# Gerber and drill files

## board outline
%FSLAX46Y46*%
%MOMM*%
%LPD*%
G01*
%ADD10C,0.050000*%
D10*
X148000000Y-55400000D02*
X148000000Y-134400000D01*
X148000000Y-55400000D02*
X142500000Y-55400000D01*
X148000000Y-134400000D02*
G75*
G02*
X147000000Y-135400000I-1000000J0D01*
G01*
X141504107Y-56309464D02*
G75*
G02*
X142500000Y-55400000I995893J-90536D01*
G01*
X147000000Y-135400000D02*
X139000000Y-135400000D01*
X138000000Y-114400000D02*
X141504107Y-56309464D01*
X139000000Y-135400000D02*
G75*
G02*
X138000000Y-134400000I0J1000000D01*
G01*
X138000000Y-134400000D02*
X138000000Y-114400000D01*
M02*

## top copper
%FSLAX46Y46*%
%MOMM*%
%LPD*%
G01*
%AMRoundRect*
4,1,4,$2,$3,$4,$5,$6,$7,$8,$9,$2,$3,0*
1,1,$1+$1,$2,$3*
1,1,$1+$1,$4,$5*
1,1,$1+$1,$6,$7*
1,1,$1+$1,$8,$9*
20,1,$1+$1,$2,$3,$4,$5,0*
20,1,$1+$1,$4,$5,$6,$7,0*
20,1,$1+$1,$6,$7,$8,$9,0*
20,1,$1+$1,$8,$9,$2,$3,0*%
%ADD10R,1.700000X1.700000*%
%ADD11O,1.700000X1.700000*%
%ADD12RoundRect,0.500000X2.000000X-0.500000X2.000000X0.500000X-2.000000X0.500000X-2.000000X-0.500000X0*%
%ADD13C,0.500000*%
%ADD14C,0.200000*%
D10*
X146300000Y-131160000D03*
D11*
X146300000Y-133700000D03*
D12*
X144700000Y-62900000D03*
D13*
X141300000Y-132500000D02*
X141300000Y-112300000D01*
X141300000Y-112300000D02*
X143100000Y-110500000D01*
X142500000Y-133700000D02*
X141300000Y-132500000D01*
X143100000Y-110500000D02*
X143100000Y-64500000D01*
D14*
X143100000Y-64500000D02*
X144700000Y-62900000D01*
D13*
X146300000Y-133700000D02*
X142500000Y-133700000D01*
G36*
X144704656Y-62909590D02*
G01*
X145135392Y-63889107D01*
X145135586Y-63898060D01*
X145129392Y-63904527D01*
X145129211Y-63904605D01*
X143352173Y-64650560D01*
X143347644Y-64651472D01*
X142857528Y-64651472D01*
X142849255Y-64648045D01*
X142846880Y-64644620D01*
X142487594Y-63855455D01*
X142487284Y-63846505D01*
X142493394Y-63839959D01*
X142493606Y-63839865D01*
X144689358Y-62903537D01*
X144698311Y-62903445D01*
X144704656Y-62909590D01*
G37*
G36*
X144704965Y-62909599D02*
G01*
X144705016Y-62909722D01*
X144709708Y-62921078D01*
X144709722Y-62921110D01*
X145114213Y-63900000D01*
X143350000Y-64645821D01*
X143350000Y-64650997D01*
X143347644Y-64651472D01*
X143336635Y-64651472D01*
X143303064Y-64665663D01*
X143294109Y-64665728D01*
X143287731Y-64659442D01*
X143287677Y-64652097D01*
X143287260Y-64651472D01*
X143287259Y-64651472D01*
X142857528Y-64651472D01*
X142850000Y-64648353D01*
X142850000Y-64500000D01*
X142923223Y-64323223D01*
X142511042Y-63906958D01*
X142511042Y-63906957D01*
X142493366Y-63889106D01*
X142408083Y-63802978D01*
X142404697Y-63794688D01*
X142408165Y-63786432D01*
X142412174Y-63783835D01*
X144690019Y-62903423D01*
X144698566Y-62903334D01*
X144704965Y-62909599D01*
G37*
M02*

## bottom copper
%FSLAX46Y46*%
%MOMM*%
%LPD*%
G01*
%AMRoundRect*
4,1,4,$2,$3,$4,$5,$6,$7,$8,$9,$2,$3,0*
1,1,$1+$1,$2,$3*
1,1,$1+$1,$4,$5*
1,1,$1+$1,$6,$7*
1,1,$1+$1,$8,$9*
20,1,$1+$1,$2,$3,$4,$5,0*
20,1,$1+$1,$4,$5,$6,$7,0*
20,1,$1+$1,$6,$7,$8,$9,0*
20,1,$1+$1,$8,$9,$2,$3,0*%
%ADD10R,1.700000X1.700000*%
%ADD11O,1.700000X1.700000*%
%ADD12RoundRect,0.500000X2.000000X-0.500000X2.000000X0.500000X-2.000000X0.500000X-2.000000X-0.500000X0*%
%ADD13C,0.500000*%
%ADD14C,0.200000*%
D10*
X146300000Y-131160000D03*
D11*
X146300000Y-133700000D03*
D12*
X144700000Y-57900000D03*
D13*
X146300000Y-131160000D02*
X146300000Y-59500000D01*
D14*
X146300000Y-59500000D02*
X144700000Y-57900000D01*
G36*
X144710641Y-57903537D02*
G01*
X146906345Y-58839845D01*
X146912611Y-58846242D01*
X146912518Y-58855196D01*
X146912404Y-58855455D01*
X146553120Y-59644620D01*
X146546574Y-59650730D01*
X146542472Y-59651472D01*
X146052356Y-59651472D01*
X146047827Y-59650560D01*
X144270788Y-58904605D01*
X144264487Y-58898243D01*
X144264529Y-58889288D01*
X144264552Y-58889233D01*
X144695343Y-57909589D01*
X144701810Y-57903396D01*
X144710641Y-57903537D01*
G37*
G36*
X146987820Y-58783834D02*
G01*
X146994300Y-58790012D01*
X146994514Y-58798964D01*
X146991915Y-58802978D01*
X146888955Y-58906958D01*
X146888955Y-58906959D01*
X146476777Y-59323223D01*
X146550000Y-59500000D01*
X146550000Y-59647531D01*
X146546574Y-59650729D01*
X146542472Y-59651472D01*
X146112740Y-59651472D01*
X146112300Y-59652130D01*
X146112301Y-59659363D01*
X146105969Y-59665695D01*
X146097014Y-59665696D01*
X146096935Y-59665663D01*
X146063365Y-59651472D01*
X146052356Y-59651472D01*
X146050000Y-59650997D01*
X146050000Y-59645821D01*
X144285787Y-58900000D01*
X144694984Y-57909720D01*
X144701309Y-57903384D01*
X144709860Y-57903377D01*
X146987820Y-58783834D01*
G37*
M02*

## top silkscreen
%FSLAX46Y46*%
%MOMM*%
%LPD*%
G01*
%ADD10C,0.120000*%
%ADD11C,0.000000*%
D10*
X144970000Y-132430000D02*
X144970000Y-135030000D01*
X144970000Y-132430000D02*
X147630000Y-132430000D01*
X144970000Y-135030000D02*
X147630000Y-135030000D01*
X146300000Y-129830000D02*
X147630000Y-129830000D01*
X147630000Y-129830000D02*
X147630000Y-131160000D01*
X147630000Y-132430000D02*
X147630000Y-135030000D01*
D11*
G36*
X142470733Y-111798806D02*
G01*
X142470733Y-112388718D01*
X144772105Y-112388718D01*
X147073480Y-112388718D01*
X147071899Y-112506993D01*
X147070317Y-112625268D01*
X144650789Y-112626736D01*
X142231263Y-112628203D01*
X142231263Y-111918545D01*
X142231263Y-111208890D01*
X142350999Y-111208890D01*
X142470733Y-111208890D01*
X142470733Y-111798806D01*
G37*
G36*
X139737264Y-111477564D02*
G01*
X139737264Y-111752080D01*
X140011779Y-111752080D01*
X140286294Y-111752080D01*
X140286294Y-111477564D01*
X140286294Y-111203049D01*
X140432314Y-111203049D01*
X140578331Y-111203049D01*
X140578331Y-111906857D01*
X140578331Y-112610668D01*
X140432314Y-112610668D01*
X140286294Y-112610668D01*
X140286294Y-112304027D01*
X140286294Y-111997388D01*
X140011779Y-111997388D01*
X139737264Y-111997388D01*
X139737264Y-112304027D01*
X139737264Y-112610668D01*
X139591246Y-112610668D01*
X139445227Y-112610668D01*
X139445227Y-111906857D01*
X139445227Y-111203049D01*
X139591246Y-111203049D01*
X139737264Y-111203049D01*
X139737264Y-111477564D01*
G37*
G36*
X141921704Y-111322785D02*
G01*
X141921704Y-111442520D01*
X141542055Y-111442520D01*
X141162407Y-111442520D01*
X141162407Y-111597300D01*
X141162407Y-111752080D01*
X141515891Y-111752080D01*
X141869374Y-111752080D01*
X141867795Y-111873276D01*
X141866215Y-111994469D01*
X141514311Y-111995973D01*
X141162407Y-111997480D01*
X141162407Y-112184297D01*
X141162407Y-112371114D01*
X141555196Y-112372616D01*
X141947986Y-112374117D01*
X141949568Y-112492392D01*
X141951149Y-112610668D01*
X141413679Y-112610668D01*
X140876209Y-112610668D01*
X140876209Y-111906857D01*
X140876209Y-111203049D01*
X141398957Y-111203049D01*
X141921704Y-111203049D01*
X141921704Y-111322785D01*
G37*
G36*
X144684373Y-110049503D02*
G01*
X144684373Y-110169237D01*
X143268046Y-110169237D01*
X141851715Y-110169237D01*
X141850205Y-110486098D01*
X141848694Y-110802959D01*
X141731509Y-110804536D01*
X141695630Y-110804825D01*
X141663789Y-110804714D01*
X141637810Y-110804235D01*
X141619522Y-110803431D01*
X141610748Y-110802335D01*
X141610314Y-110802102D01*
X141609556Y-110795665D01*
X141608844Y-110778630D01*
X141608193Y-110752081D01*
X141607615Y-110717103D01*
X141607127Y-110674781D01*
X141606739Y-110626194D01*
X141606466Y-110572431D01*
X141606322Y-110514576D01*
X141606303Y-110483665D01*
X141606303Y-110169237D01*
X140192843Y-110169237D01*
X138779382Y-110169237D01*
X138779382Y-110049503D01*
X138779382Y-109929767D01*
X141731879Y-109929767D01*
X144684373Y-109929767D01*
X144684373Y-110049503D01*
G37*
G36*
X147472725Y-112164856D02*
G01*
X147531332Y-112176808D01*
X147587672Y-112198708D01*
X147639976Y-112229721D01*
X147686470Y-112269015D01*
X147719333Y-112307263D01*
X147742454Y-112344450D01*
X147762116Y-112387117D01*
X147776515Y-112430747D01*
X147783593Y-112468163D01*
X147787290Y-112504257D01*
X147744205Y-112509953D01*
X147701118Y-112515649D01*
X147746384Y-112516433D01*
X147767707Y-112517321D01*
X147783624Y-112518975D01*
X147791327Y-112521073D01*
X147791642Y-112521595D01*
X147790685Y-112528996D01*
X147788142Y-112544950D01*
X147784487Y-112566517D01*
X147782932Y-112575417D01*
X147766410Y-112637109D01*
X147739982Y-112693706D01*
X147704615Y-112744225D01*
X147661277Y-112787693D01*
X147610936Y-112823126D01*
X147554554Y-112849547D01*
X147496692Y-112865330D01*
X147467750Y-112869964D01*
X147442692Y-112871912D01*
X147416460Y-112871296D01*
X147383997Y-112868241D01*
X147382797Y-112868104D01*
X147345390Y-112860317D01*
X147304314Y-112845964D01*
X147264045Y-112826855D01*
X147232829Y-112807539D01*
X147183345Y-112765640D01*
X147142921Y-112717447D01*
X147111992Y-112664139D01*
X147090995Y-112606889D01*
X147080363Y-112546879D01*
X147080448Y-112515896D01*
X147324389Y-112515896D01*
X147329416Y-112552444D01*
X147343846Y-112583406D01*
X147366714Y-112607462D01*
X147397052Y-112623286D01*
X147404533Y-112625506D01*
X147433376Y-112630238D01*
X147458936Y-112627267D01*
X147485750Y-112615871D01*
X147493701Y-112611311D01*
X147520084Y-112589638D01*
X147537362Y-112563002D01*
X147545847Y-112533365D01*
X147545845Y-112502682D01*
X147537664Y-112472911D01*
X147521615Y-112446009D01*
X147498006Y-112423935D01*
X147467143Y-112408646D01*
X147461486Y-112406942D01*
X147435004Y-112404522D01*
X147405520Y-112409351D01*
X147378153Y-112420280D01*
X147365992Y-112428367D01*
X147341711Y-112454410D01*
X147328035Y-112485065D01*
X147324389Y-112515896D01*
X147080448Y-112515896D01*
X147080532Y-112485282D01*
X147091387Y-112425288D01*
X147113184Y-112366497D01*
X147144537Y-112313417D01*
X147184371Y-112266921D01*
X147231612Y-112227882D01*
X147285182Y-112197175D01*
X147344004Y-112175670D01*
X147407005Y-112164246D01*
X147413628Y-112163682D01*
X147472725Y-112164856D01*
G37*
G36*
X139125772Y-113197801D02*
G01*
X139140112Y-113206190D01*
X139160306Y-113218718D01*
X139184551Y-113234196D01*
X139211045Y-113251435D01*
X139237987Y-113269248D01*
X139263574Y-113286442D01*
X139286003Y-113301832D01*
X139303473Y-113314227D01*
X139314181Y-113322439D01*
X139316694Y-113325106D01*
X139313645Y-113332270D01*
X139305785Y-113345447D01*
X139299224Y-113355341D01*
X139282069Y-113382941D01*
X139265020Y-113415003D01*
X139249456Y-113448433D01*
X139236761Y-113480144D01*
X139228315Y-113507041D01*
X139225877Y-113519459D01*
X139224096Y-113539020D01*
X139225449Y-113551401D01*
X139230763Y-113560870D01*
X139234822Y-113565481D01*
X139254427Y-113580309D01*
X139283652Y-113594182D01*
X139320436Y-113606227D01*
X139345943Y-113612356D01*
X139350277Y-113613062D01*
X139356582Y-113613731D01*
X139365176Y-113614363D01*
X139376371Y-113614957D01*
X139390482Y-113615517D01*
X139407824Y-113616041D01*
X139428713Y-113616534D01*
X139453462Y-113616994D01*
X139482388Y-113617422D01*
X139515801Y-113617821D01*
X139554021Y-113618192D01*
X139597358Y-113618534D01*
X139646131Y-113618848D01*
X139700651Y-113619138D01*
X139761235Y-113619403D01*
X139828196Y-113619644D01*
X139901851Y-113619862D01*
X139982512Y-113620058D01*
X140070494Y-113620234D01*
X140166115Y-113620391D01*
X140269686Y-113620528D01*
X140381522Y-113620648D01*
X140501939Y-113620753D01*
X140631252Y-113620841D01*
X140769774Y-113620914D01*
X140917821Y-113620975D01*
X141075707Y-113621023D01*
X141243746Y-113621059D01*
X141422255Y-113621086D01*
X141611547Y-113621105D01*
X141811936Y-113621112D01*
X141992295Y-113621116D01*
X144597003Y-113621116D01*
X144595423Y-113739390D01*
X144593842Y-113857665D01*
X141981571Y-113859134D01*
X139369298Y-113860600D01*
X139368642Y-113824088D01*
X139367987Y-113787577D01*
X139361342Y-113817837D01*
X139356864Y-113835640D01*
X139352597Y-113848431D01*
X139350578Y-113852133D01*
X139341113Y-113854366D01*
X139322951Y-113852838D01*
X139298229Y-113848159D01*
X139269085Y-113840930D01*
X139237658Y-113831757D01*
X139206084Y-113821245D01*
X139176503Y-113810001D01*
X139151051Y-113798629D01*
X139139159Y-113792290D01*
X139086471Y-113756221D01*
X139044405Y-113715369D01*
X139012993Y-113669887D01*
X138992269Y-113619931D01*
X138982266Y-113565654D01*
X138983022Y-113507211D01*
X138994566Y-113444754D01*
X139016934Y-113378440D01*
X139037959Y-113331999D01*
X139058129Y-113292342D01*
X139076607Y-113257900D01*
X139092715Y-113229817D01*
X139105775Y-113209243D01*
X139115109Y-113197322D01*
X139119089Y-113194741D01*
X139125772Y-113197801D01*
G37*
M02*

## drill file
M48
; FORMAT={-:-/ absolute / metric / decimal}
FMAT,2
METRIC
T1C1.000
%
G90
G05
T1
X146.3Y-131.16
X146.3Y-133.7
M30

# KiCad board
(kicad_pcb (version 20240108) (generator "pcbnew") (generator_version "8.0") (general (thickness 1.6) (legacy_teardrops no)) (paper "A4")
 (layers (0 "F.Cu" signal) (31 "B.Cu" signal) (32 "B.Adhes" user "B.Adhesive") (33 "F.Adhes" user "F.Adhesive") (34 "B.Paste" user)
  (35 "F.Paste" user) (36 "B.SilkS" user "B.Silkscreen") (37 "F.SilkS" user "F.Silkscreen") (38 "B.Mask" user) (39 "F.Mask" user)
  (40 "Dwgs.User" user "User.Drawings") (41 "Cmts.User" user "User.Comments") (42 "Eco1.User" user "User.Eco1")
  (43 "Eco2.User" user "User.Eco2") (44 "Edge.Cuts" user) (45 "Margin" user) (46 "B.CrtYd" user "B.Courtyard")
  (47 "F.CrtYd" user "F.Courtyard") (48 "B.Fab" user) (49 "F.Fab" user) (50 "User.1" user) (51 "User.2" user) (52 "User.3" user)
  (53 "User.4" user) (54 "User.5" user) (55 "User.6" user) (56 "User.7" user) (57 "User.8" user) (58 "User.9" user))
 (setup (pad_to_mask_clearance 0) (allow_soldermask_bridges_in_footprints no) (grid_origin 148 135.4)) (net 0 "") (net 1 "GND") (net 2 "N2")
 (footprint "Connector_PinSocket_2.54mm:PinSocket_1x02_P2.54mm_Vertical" (layer "F.Cu") (at 146.3 131.16)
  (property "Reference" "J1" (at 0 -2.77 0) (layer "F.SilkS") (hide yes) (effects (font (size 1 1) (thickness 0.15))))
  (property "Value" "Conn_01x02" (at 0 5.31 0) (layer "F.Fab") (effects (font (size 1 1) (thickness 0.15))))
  (fp_line (start -1.33 1.27) (end -1.33 3.87) (stroke (width 0.12) (type solid)) (layer "F.SilkS"))
  (fp_line (start -1.33 1.27) (end 1.33 1.27) (stroke (width 0.12) (type solid)) (layer "F.SilkS"))
  (fp_line (start -1.33 3.87) (end 1.33 3.87) (stroke (width 0.12) (type solid)) (layer "F.SilkS"))
  (fp_line (start 0 -1.33) (end 1.33 -1.33) (stroke (width 0.12) (type solid)) (layer "F.SilkS"))
  (fp_line (start 1.33 -1.33) (end 1.33 0) (stroke (width 0.12) (type solid)) (layer "F.SilkS"))
  (fp_line (start 1.33 1.27) (end 1.33 3.87) (stroke (width 0.12) (type solid)) (layer "F.SilkS"))
  (pad "1" thru_hole rect (at 0 0) (size 1.7 1.7) (drill 1) (layers "*.Cu" "*.Mask") (remove_unused_layers no) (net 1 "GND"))
  (pad "2" thru_hole oval (at 0 2.54) (size 1.7 1.7) (drill 1) (layers "*.Cu" "*.Mask") (remove_unused_layers no) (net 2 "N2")))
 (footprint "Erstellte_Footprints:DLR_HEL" (layer "F.Cu") (at 143.3 111.9)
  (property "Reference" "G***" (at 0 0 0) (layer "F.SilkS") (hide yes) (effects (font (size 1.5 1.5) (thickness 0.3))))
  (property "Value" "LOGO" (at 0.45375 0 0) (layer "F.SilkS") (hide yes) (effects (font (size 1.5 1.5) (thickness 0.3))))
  (fp_poly
   (pts (xy -0.829267 -0.101194) (xy -0.829267 0.488718) (xy 1.472105 0.488718) (xy 3.77348 0.488718) (xy 3.771899 0.606993)
    (xy 3.770317 0.725268) (xy 1.350789 0.726736) (xy -1.068737 0.728203) (xy -1.068737 0.018545) (xy -1.068737 -0.69111)
    (xy -0.949001 -0.69111) (xy -0.829267 -0.69111))
   (stroke (width 0) (type solid)) (fill solid) (layer "F.SilkS"))
  (fp_poly
   (pts (xy -3.562736 -0.422436) (xy -3.562736 -0.14792) (xy -3.288221 -0.14792) (xy -3.013706 -0.14792) (xy -3.013706 -0.422436)
    (xy -3.013706 -0.696951) (xy -2.867686 -0.696951) (xy -2.721669 -0.696951) (xy -2.721669 0.006857) (xy -2.721669 0.710668)
    (xy -2.867686 0.710668) (xy -3.013706 0.710668) (xy -3.013706 0.404027) (xy -3.013706 0.097388) (xy -3.288221 0.097388)
    (xy -3.562736 0.097388) (xy -3.562736 0.404027) (xy -3.562736 0.710668) (xy -3.708754 0.710668) (xy -3.854773 0.710668)
    (xy -3.854773 0.006857) (xy -3.854773 -0.696951) (xy -3.708754 -0.696951) (xy -3.562736 -0.696951))
   (stroke (width 0) (type solid)) (fill solid) (layer "F.SilkS"))
  (fp_poly
   (pts (xy -1.378296 -0.577215) (xy -1.378296 -0.45748) (xy -1.757945 -0.45748) (xy -2.137593 -0.45748) (xy -2.137593 -0.3027)
    (xy -2.137593 -0.14792) (xy -1.784109 -0.14792) (xy -1.430626 -0.14792) (xy -1.432205 -0.026724) (xy -1.433785 0.094469)
    (xy -1.785689 0.095973) (xy -2.137593 0.09748) (xy -2.137593 0.284297) (xy -2.137593 0.471114) (xy -1.744804 0.472616)
    (xy -1.352014 0.474117) (xy -1.350432 0.592392) (xy -1.348851 0.710668) (xy -1.886321 0.710668) (xy -2.423791 0.710668)
    (xy -2.423791 0.006857) (xy -2.423791 -0.696951) (xy -1.901043 -0.696951) (xy -1.378296 -0.696951))
   (stroke (width 0) (type solid)) (fill solid) (layer "F.SilkS"))
  (fp_poly
   (pts (xy 1.384373 -1.850497) (xy 1.384373 -1.730763) (xy -0.031954 -1.730763) (xy -1.448285 -1.730763) (xy -1.449795 -1.413902)
    (xy -1.451306 -1.097041) (xy -1.568491 -1.095464) (xy -1.60437 -1.095175) (xy -1.636211 -1.095286) (xy -1.66219 -1.095765)
    (xy -1.680478 -1.096569) (xy -1.689252 -1.097665) (xy -1.689686 -1.097898) (xy -1.690444 -1.104335) (xy -1.691156 -1.12137)
    (xy -1.691807 -1.147919) (xy -1.692385 -1.182897) (xy -1.692873 -1.225219) (xy -1.693261 -1.273806) (xy -1.693534 -1.327569)
    (xy -1.693678 -1.385424) (xy -1.693697 -1.416335) (xy -1.693697 -1.730763) (xy -3.107157 -1.730763) (xy -4.520618 -1.730763)
    (xy -4.520618 -1.850497) (xy -4.520618 -1.970233) (xy -1.568121 -1.970233) (xy 1.384373 -1.970233))
   (stroke (width 0) (type solid)) (fill solid) (layer "F.SilkS"))
  (fp_poly
   (pts (xy 4.172725 0.264856) (xy 4.231332 0.276808) (xy 4.287672 0.298708) (xy 4.339976 0.329721) (xy 4.38647 0.369015)
    (xy 4.419333 0.407263) (xy 4.442454 0.44445) (xy 4.462116 0.487117) (xy 4.476515 0.530747) (xy 4.483593 0.568163) (xy 4.48729 0.604257)
    (xy 4.444205 0.609953) (xy 4.401118 0.615649) (xy 4.446384 0.616433) (xy 4.467707 0.617321) (xy 4.483624 0.618975)
    (xy 4.491327 0.621073) (xy 4.491642 0.621595) (xy 4.490685 0.628996) (xy 4.488142 0.64495) (xy 4.484487 0.666517) (xy 4.482932 0.675417)
    (xy 4.46641 0.737109) (xy 4.439982 0.793706) (xy 4.404615 0.844225) (xy 4.361277 0.887693) (xy 4.310936 0.923126) (xy 4.254554 0.949547)
    (xy 4.196692 0.96533) (xy 4.16775 0.969964) (xy 4.142692 0.971912) (xy 4.11646 0.971296) (xy 4.083997 0.968241) (xy 4.082797 0.968104)
    (xy 4.04539 0.960317) (xy 4.004314 0.945964) (xy 3.964045 0.926855) (xy 3.932829 0.907539) (xy 3.883345 0.86564) (xy 3.842921 0.817447)
    (xy 3.811992 0.764139) (xy 3.790995 0.706889) (xy 3.780363 0.646879) (xy 3.780448 0.615896) (xy 4.024389 0.615896)
    (xy 4.029416 0.652444) (xy 4.043846 0.683406) (xy 4.066714 0.707462) (xy 4.097052 0.723286) (xy 4.104533 0.725506)
    (xy 4.133376 0.730238) (xy 4.158936 0.727267) (xy 4.18575 0.715871) (xy 4.193701 0.711311) (xy 4.220084 0.689638) (xy 4.237362 0.663002)
    (xy 4.245847 0.633365) (xy 4.245845 0.602682) (xy 4.237664 0.572911) (xy 4.221615 0.546009) (xy 4.198006 0.523935)
    (xy 4.167143 0.508646) (xy 4.161486 0.506942) (xy 4.135004 0.504522) (xy 4.10552 0.509351) (xy 4.078153 0.52028) (xy 4.065992 0.528367)
    (xy 4.041711 0.55441) (xy 4.028035 0.585065) (xy 4.024389 0.615896) (xy 3.780448 0.615896) (xy 3.780532 0.585282) (xy 3.791387 0.525288)
    (xy 3.813184 0.466497) (xy 3.844537 0.413417) (xy 3.884371 0.366921) (xy 3.931612 0.327882) (xy 3.985182 0.297175) (xy 4.044004 0.27567)
    (xy 4.107005 0.264246) (xy 4.113628 0.263682))
   (stroke (width 0) (type solid)) (fill solid) (layer "F.SilkS"))
  (fp_poly
   (pts (xy -4.174228 1.297801) (xy -4.159888 1.30619) (xy -4.139694 1.318718) (xy -4.115449 1.334196) (xy -4.088955 1.351435)
    (xy -4.062013 1.369248) (xy -4.036426 1.386442) (xy -4.013997 1.401832) (xy -3.996527 1.414227) (xy -3.985819 1.422439)
    (xy -3.983306 1.425106) (xy -3.986355 1.43227) (xy -3.994215 1.445447) (xy -4.000776 1.455341) (xy -4.017931 1.482941)
    (xy -4.03498 1.515003) (xy -4.050544 1.548433) (xy -4.063239 1.580144) (xy -4.071685 1.607041) (xy -4.074123 1.619459)
    (xy -4.075904 1.63902) (xy -4.074551 1.651401) (xy -4.069237 1.66087) (xy -4.065178 1.665481) (xy -4.045573 1.680309)
    (xy -4.016348 1.694182) (xy -3.979564 1.706227) (xy -3.954057 1.712356) (xy -3.949723 1.713062) (xy -3.943418 1.713731)
    (xy -3.934824 1.714363) (xy -3.923629 1.714957) (xy -3.909518 1.715517) (xy -3.892176 1.716041) (xy -3.871287 1.716534)
    (xy -3.846538 1.716994) (xy -3.817612 1.717422) (xy -3.784199 1.717821) (xy -3.745979 1.718192) (xy -3.702642 1.718534)
    (xy -3.653869 1.718848) (xy -3.599349 1.719138) (xy -3.538765 1.719403) (xy -3.471804 1.719644) (xy -3.398149 1.719862)
    (xy -3.317488 1.720058) (xy -3.229506 1.720234) (xy -3.133885 1.720391) (xy -3.030314 1.720528) (xy -2.918478 1.720648)
    (xy -2.798061 1.720753) (xy -2.668748 1.720841) (xy -2.530226 1.720914) (xy -2.382179 1.720975) (xy -2.224293 1.721023)
    (xy -2.056254 1.721059) (xy -1.877745 1.721086) (xy -1.688453 1.721105) (xy -1.488064 1.721112) (xy -1.307705 1.721116)
    (xy 1.297003 1.721116) (xy 1.295423 1.83939) (xy 1.293842 1.957665) (xy -1.318429 1.959134) (xy -3.930702 1.9606)
    (xy -3.931358 1.924088) (xy -3.932013 1.887577) (xy -3.938658 1.917837) (xy -3.943136 1.93564) (xy -3.947403 1.948431)
    (xy -3.949422 1.952133) (xy -3.958887 1.954366) (xy -3.977049 1.952838) (xy -4.001771 1.948159) (xy -4.030915 1.94093)
    (xy -4.062342 1.931757) (xy -4.093916 1.921245) (xy -4.123497 1.910001) (xy -4.148949 1.898629) (xy -4.160841 1.89229)
    (xy -4.213529 1.856221) (xy -4.255595 1.815369) (xy -4.287007 1.769887) (xy -4.307731 1.719931) (xy -4.317734 1.665654)
    (xy -4.316978 1.607211) (xy -4.305434 1.544754) (xy -4.283066 1.47844) (xy -4.262041 1.431999) (xy -4.241871 1.392342)
    (xy -4.223393 1.3579) (xy -4.207285 1.329817) (xy -4.194225 1.309243) (xy -4.184891 1.297322) (xy -4.180911 1.294741))
   (stroke (width 0) (type solid)) (fill solid) (layer "F.SilkS")))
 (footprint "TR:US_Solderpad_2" (layer "F.Cu") (at 144.7 60.4 90)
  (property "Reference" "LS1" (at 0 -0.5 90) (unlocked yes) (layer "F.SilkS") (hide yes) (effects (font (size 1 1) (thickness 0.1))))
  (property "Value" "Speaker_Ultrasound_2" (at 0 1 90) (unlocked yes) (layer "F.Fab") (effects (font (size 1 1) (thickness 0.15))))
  (pad "1" smd roundrect (at -2.5 0 90) (size 2 5) (layers "F.Cu" "F.Paste" "F.Mask") (roundrect_rratio 0.25) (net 2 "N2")
   (thermal_bridge_angle 45)
   (teardrops (best_length_ratio 0.5) (max_length 1) (best_width_ratio 1) (max_width 2) (curve_points 0) (filter_ratio 0.9) (enabled yes)
    (allow_two_segments yes) (prefer_zone_connections yes)))
  (pad "2" smd roundrect (at 2.5 0 90) (size 2 5) (layers "B.Cu" "B.Paste" "B.Mask") (roundrect_rratio 0.25) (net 1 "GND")
   (thermal_bridge_angle 45)
   (teardrops (best_length_ratio 0.5) (max_length 1) (best_width_ratio 1) (max_width 2) (curve_points 0) (filter_ratio 0.9) (enabled yes)
    (allow_two_segments yes) (prefer_zone_connections yes))))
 (gr_line (start 148 55.4) (end 148 134.4) (stroke (width 0.05) (type default)) (layer "Edge.Cuts"))
 (gr_line (start 148 55.4) (end 142.5 55.4) (stroke (width 0.05) (type default)) (layer "Edge.Cuts"))
 (gr_arc (start 148 134.4) (mid 147.707107 135.107107) (end 147 135.4) (stroke (width 0.05) (type default)) (layer "Edge.Cuts"))
 (gr_arc (start 141.504107 56.309464) (mid 141.825662 55.661577) (end 142.5 55.4) (stroke (width 0.05) (type default)) (layer "Edge.Cuts"))
 (gr_line (start 147 135.4) (end 139 135.4) (stroke (width 0.05) (type default)) (layer "Edge.Cuts"))
 (gr_line (start 138 114.4) (end 141.504107 56.309464) (stroke (width 0.05) (type default)) (layer "Edge.Cuts"))
 (gr_arc (start 139 135.4) (mid 138.292893 135.107107) (end 138 134.4) (stroke (width 0.05) (type default)) (layer "Edge.Cuts"))
 (gr_line (start 138 134.4) (end 138 114.4) (stroke (width 0.05) (type default)) (layer "Edge.Cuts"))
 (segment (start 141.3 132.5) (end 141.3 112.3) (width 0.5) (layer "F.Cu") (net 2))
 (segment (start 141.3 112.3) (end 143.1 110.5) (width 0.5) (layer "F.Cu") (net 2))
 (segment (start 142.5 133.7) (end 141.3 132.5) (width 0.5) (layer "F.Cu") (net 2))
 (segment (start 143.1 110.5) (end 143.1 64.5) (width 0.5) (layer "F.Cu") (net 2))
 (segment (start 143.1 64.5) (end 144.7 62.9) (width 0.2) (layer "F.Cu") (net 2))
 (segment (start 146.3 133.7) (end 142.5 133.7) (width 0.5) (layer "F.Cu") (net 2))
 (segment (start 146.3 131.16) (end 146.3 59.5) (width 0.5) (layer "B.Cu") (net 1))
 (segment (start 146.3 59.5) (end 144.7 57.9) (width 0.2) (layer "B.Cu") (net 1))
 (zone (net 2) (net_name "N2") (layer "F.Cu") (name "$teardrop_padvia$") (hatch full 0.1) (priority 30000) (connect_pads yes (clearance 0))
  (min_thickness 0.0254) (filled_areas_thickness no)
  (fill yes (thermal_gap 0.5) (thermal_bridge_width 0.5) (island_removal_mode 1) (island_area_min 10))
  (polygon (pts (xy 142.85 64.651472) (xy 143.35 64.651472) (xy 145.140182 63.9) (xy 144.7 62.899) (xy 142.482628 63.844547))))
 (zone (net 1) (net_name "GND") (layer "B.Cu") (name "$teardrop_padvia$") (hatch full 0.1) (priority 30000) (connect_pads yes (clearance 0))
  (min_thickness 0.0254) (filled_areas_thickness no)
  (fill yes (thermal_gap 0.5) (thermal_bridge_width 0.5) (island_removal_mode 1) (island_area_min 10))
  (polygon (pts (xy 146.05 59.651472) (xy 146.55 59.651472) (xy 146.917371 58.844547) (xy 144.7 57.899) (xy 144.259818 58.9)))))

